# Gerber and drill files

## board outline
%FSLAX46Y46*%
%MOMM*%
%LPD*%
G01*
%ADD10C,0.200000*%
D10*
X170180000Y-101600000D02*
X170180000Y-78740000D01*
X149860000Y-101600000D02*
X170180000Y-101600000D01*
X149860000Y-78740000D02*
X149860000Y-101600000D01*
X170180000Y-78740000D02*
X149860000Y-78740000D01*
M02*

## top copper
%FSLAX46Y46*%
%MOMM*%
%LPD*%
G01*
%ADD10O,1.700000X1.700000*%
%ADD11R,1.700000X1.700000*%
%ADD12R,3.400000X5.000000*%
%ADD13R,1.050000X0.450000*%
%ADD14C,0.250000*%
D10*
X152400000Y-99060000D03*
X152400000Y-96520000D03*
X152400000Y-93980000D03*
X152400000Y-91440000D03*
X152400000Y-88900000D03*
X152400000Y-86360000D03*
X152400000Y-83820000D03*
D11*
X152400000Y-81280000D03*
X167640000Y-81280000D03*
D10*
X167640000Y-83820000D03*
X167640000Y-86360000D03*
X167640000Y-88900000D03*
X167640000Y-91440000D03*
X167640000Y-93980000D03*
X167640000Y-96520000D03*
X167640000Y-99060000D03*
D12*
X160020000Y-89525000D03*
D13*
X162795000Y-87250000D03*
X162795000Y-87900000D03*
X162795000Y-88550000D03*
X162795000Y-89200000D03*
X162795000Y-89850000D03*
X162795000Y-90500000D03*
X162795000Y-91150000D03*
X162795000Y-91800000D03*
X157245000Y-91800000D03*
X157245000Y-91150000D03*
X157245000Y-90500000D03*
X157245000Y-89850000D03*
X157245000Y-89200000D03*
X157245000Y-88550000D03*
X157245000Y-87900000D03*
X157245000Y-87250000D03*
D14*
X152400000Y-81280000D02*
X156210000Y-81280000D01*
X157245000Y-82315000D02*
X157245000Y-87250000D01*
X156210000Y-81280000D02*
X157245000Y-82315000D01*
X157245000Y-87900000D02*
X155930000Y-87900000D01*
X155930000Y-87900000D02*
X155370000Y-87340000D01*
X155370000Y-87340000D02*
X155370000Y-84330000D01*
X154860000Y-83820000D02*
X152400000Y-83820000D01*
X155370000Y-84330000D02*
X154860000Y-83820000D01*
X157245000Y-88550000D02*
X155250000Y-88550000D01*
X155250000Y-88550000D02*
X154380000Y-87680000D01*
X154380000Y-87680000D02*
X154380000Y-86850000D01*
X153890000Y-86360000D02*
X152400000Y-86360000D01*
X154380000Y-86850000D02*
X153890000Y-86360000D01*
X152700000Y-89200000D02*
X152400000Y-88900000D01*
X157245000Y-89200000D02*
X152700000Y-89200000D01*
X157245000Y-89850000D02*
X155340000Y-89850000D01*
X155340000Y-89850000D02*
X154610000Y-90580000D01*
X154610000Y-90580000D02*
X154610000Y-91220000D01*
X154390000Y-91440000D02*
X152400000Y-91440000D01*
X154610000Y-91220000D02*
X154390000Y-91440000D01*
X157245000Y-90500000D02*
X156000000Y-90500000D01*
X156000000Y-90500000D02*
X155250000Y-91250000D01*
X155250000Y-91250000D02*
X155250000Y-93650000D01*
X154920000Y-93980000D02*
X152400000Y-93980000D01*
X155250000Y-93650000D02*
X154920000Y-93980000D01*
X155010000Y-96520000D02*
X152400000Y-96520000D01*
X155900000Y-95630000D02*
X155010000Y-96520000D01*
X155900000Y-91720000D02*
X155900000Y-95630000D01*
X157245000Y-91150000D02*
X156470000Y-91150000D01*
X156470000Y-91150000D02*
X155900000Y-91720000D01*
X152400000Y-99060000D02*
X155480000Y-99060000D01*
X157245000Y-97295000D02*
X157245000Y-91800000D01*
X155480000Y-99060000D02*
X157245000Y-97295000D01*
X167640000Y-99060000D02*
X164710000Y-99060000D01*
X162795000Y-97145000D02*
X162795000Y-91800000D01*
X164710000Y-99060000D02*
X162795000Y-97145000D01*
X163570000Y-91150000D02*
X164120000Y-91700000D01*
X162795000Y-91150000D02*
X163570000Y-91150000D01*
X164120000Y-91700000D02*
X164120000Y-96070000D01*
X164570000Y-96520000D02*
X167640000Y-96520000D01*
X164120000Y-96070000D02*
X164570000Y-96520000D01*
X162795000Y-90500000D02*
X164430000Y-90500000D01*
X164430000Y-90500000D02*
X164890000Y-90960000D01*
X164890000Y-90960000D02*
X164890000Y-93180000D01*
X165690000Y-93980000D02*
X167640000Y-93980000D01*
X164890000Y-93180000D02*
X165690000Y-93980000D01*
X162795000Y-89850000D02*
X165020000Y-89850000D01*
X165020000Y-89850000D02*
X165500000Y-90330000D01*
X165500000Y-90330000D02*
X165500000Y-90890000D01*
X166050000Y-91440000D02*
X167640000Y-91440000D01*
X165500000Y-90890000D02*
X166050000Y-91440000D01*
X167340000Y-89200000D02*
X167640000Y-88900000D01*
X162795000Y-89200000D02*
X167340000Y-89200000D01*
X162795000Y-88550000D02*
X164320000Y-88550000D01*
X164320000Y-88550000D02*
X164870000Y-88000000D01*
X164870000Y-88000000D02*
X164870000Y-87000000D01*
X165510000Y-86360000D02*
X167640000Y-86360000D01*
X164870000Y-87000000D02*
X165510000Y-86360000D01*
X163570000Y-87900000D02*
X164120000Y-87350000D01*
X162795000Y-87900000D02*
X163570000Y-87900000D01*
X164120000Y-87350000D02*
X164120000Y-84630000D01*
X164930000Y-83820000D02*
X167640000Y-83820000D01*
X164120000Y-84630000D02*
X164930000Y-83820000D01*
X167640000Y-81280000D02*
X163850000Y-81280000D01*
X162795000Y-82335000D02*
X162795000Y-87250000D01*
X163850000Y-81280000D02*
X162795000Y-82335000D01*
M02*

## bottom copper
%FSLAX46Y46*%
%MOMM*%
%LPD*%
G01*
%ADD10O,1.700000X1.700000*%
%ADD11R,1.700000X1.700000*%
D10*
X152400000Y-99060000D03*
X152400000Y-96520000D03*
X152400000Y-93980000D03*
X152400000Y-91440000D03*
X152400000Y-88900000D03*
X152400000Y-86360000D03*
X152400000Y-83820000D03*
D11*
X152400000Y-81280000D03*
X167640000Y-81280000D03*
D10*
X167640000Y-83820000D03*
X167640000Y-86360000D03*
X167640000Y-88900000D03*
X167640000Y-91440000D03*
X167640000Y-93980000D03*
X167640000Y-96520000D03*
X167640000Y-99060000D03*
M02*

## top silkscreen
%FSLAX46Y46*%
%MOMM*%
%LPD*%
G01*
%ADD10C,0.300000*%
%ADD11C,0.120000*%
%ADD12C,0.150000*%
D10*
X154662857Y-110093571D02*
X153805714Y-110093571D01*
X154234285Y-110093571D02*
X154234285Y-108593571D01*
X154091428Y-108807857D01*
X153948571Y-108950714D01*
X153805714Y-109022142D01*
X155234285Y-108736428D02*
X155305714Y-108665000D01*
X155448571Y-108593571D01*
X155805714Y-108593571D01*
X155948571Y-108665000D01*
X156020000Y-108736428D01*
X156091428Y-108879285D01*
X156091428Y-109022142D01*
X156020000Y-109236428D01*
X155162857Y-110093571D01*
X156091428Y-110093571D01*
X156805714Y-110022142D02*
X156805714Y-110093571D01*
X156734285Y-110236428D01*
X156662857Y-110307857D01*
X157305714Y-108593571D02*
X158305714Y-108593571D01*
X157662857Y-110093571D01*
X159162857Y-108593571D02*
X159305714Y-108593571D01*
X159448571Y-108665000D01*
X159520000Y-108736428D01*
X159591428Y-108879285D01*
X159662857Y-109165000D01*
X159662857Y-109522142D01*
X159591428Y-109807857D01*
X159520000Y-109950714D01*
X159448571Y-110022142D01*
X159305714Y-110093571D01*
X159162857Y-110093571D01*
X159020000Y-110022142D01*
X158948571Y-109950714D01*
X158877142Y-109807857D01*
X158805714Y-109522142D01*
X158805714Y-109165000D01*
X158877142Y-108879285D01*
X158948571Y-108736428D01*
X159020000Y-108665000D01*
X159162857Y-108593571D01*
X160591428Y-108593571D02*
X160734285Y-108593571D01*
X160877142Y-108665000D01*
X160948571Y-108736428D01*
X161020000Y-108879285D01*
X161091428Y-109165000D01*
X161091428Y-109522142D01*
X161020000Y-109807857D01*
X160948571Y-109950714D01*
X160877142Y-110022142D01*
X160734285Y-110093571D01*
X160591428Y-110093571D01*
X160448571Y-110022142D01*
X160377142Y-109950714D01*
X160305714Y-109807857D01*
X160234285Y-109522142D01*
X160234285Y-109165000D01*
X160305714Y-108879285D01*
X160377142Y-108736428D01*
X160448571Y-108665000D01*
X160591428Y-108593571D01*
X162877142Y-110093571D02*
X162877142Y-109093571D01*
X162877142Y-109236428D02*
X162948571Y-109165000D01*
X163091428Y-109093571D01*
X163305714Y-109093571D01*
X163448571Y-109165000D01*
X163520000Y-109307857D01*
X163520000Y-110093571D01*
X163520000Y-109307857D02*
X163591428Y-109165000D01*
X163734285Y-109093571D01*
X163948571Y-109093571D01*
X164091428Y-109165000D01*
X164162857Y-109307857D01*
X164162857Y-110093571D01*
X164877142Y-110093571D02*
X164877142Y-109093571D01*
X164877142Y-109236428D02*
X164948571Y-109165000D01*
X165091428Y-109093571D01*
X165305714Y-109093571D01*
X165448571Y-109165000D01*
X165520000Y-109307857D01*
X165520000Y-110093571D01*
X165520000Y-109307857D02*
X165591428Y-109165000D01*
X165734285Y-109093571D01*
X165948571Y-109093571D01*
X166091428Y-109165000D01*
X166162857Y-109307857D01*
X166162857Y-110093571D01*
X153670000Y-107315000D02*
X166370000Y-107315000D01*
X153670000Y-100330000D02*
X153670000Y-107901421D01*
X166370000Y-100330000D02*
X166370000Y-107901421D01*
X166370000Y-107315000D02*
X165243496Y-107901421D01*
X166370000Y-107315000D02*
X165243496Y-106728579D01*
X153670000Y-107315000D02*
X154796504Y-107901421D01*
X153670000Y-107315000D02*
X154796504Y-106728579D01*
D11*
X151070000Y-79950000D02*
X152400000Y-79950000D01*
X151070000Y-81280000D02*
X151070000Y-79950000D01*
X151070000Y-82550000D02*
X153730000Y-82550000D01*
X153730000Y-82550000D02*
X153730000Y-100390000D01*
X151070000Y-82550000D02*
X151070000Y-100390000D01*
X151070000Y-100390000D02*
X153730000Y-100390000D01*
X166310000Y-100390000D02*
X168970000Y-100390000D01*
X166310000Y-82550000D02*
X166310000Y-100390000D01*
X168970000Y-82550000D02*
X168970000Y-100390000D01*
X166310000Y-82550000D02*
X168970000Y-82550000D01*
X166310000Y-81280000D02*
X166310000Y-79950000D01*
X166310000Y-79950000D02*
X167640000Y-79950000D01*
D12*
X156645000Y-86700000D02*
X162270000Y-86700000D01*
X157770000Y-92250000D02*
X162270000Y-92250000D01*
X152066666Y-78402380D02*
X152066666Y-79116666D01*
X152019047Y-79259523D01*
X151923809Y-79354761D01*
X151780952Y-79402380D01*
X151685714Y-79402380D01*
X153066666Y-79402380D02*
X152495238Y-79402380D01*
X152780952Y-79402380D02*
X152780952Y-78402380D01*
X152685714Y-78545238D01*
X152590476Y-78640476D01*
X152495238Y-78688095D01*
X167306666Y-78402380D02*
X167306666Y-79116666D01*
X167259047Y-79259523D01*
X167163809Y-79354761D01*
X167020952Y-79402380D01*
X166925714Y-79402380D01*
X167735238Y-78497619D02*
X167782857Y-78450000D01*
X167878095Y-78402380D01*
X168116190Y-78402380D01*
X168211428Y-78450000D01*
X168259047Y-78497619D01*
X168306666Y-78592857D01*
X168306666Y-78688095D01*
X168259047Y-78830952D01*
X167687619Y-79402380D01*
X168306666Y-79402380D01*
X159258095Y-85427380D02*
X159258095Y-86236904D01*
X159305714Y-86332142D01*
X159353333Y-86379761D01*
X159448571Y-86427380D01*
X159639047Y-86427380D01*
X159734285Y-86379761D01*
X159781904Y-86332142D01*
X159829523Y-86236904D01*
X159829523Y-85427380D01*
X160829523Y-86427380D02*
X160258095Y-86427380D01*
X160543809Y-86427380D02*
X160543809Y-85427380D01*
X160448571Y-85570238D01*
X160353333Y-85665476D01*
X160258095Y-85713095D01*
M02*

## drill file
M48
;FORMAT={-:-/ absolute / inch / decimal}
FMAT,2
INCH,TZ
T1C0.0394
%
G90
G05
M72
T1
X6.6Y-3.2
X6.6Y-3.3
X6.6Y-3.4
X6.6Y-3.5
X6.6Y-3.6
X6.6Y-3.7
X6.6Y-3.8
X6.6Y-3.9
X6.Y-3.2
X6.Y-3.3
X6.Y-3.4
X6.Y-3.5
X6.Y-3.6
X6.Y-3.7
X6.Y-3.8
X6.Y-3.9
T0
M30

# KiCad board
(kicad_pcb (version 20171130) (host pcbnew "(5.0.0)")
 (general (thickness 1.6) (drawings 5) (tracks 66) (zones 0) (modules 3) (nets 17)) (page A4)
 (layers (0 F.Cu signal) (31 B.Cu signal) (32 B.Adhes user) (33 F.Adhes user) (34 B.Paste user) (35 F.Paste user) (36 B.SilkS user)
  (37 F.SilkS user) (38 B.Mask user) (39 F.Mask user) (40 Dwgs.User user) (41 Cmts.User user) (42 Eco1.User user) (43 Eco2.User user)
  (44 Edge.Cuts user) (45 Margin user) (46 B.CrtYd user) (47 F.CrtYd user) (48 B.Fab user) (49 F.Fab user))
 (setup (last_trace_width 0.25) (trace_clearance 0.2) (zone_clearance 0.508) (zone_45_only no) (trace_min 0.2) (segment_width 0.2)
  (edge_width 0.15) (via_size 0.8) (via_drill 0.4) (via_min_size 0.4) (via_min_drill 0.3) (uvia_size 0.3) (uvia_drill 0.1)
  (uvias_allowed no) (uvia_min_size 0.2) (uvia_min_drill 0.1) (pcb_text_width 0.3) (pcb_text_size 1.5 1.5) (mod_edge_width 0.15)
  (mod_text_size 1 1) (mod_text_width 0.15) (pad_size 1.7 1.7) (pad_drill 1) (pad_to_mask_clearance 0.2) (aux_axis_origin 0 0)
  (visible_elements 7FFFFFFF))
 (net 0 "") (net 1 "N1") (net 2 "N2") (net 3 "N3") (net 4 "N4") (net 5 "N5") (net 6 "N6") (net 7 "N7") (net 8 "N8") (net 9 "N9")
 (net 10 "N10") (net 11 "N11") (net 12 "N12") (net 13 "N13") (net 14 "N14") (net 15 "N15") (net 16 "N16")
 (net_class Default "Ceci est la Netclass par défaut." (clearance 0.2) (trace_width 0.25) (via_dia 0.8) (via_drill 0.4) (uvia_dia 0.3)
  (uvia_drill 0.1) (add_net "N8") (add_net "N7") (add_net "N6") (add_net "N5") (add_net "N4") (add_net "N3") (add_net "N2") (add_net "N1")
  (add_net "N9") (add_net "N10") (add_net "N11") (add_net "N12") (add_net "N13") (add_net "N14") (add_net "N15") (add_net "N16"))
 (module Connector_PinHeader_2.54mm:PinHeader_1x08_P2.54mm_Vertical (layer F.Cu) (at 152.4 81.28)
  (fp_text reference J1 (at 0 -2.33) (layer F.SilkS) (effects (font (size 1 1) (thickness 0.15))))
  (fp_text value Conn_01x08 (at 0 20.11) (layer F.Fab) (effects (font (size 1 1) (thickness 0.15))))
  (fp_line (start -1.33 -1.33) (end 0 -1.33) (layer F.SilkS) (width 0.12))
  (fp_line (start -1.33 0) (end -1.33 -1.33) (layer F.SilkS) (width 0.12))
  (fp_line (start -1.33 1.27) (end 1.33 1.27) (layer F.SilkS) (width 0.12))
  (fp_line (start 1.33 1.27) (end 1.33 19.11) (layer F.SilkS) (width 0.12))
  (fp_line (start -1.33 1.27) (end -1.33 19.11) (layer F.SilkS) (width 0.12))
  (fp_line (start -1.33 19.11) (end 1.33 19.11) (layer F.SilkS) (width 0.12))
  (pad 8 thru_hole oval (at 0 17.78) (size 1.7 1.7) (drill 1) (layers *.Cu *.Mask) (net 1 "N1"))
  (pad 7 thru_hole oval (at 0 15.24) (size 1.7 1.7) (drill 1) (layers *.Cu *.Mask) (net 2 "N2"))
  (pad 6 thru_hole oval (at 0 12.7) (size 1.7 1.7) (drill 1) (layers *.Cu *.Mask) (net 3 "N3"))
  (pad 5 thru_hole oval (at 0 10.16) (size 1.7 1.7) (drill 1) (layers *.Cu *.Mask) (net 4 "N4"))
  (pad 4 thru_hole oval (at 0 7.62) (size 1.7 1.7) (drill 1) (layers *.Cu *.Mask) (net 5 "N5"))
  (pad 3 thru_hole oval (at 0 5.08) (size 1.7 1.7) (drill 1) (layers *.Cu *.Mask) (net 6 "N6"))
  (pad 2 thru_hole oval (at 0 2.54) (size 1.7 1.7) (drill 1) (layers *.Cu *.Mask) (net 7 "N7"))
  (pad 1 thru_hole rect (at 0 0) (size 1.7 1.7) (drill 1) (layers *.Cu *.Mask) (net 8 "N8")))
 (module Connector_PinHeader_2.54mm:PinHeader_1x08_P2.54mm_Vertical (layer F.Cu) (at 167.64 81.28)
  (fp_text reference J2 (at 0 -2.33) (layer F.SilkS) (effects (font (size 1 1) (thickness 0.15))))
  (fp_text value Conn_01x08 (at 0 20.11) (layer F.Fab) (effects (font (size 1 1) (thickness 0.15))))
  (fp_line (start -1.33 19.11) (end 1.33 19.11) (layer F.SilkS) (width 0.12))
  (fp_line (start -1.33 1.27) (end -1.33 19.11) (layer F.SilkS) (width 0.12))
  (fp_line (start 1.33 1.27) (end 1.33 19.11) (layer F.SilkS) (width 0.12))
  (fp_line (start -1.33 1.27) (end 1.33 1.27) (layer F.SilkS) (width 0.12))
  (fp_line (start -1.33 0) (end -1.33 -1.33) (layer F.SilkS) (width 0.12))
  (fp_line (start -1.33 -1.33) (end 0 -1.33) (layer F.SilkS) (width 0.12))
  (pad 1 thru_hole rect (at 0 0) (size 1.7 1.7) (drill 1) (layers *.Cu *.Mask) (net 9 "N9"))
  (pad 2 thru_hole oval (at 0 2.54) (size 1.7 1.7) (drill 1) (layers *.Cu *.Mask) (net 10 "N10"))
  (pad 3 thru_hole oval (at 0 5.08) (size 1.7 1.7) (drill 1) (layers *.Cu *.Mask) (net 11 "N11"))
  (pad 4 thru_hole oval (at 0 7.62) (size 1.7 1.7) (drill 1) (layers *.Cu *.Mask) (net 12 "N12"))
  (pad 5 thru_hole oval (at 0 10.16) (size 1.7 1.7) (drill 1) (layers *.Cu *.Mask) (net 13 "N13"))
  (pad 6 thru_hole oval (at 0 12.7) (size 1.7 1.7) (drill 1) (layers *.Cu *.Mask) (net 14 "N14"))
  (pad 7 thru_hole oval (at 0 15.24) (size 1.7 1.7) (drill 1) (layers *.Cu *.Mask) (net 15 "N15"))
  (pad 8 thru_hole oval (at 0 17.78) (size 1.7 1.7) (drill 1) (layers *.Cu *.Mask) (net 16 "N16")))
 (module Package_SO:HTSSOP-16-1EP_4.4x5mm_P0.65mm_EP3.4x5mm (layer F.Cu) (at 160.02 89.525)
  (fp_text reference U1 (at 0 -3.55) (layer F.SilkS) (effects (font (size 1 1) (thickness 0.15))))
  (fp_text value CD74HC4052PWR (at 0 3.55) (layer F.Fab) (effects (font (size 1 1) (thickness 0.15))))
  (fp_line (start -3.375 -2.825) (end 2.25 -2.825) (layer F.SilkS) (width 0.15))
  (fp_line (start -2.25 2.725) (end 2.25 2.725) (layer F.SilkS) (width 0.15))
  (pad "" smd rect (at -1.1334 1.875) (size 0.88 1.05) (layers F.Paste))
  (pad "" smd rect (at 0 1.875) (size 0.88 1.05) (layers F.Paste))
  (pad "" smd rect (at 1.1334 1.875) (size 0.88 1.05) (layers F.Paste))
  (pad "" smd rect (at -1.1334 0.625) (size 0.88 1.05) (layers F.Paste))
  (pad "" smd rect (at 0 0.625) (size 0.88 1.05) (layers F.Paste))
  (pad "" smd rect (at 1.1334 0.625) (size 0.88 1.05) (layers F.Paste))
  (pad "" smd rect (at -1.1334 -0.625) (size 0.88 1.05) (layers F.Paste))
  (pad "" smd rect (at 0 -0.625) (size 0.88 1.05) (layers F.Paste))
  (pad "" smd rect (at 1.1334 -0.625) (size 0.88 1.05) (layers F.Paste))
  (pad "" smd rect (at 1.1334 -1.875) (size 0.88 1.05) (layers F.Paste))
  (pad "" smd rect (at 0 -1.875) (size 0.88 1.05) (layers F.Paste))
  (pad "" smd rect (at -1.1334 -1.875) (size 0.88 1.05) (layers F.Paste)) (pad 17 smd rect (at 0 0) (size 3.4 5) (layers F.Cu F.Mask))
  (pad 16 smd rect (at 2.775 -2.275) (size 1.05 0.45) (layers F.Cu F.Paste F.Mask) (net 9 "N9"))
  (pad 15 smd rect (at 2.775 -1.625) (size 1.05 0.45) (layers F.Cu F.Paste F.Mask) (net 10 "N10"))
  (pad 14 smd rect (at 2.775 -0.975) (size 1.05 0.45) (layers F.Cu F.Paste F.Mask) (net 11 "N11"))
  (pad 13 smd rect (at 2.775 -0.325) (size 1.05 0.45) (layers F.Cu F.Paste F.Mask) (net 12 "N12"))
  (pad 12 smd rect (at 2.775 0.325) (size 1.05 0.45) (layers F.Cu F.Paste F.Mask) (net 13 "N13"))
  (pad 11 smd rect (at 2.775 0.975) (size 1.05 0.45) (layers F.Cu F.Paste F.Mask) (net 14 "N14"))
  (pad 10 smd rect (at 2.775 1.625) (size 1.05 0.45) (layers F.Cu F.Paste F.Mask) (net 15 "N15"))
  (pad 9 smd rect (at 2.775 2.275) (size 1.05 0.45) (layers F.Cu F.Paste F.Mask) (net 16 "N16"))
  (pad 8 smd rect (at -2.775 2.275) (size 1.05 0.45) (layers F.Cu F.Paste F.Mask) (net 1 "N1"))
  (pad 7 smd rect (at -2.775 1.625) (size 1.05 0.45) (layers F.Cu F.Paste F.Mask) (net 2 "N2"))
  (pad 6 smd rect (at -2.775 0.975) (size 1.05 0.45) (layers F.Cu F.Paste F.Mask) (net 3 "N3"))
  (pad 5 smd rect (at -2.775 0.325) (size 1.05 0.45) (layers F.Cu F.Paste F.Mask) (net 4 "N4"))
  (pad 4 smd rect (at -2.775 -0.325) (size 1.05 0.45) (layers F.Cu F.Paste F.Mask) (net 5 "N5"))
  (pad 3 smd rect (at -2.775 -0.975) (size 1.05 0.45) (layers F.Cu F.Paste F.Mask) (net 6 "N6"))
  (pad 2 smd rect (at -2.775 -1.625) (size 1.05 0.45) (layers F.Cu F.Paste F.Mask) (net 7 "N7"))
  (pad 1 smd rect (at -2.775 -2.275) (size 1.05 0.45) (layers F.Cu F.Paste F.Mask) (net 8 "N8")))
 (gr_line (start 170.18 101.6) (end 170.18 78.74) (layer Edge.Cuts) (width 0.2))
 (gr_line (start 149.86 101.6) (end 170.18 101.6) (layer Edge.Cuts) (width 0.2))
 (gr_line (start 149.86 78.74) (end 149.86 101.6) (layer Edge.Cuts) (width 0.2))
 (gr_line (start 170.18 78.74) (end 149.86 78.74) (layer Edge.Cuts) (width 0.2))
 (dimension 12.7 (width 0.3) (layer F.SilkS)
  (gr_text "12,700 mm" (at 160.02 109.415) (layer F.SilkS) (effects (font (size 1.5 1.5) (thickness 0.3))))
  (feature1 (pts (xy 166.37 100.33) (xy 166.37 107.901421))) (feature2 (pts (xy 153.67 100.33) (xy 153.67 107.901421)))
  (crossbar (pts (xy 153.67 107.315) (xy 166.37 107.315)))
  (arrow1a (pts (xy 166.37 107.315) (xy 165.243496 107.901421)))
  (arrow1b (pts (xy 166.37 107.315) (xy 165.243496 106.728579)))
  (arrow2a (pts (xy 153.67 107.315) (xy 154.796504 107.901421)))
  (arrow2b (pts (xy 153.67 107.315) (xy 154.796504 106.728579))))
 (segment (start 152.4 81.28) (end 156.21 81.28) (width 0.25) (layer F.Cu) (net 8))
 (segment (start 157.245 82.315) (end 157.245 87.25) (width 0.25) (layer F.Cu) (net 8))
 (segment (start 156.21 81.28) (end 157.245 82.315) (width 0.25) (layer F.Cu) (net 8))
 (segment (start 157.245 87.9) (end 155.93 87.9) (width 0.25) (layer F.Cu) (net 7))
 (segment (start 155.93 87.9) (end 155.37 87.34) (width 0.25) (layer F.Cu) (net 7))
 (segment (start 155.37 87.34) (end 155.37 84.33) (width 0.25) (layer F.Cu) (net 7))
 (segment (start 154.86 83.82) (end 152.4 83.82) (width 0.25) (layer F.Cu) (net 7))
 (segment (start 155.37 84.33) (end 154.86 83.82) (width 0.25) (layer F.Cu) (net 7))
 (segment (start 157.245 88.55) (end 155.25 88.55) (width 0.25) (layer F.Cu) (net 6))
 (segment (start 155.25 88.55) (end 154.38 87.68) (width 0.25) (layer F.Cu) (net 6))
 (segment (start 154.38 87.68) (end 154.38 86.85) (width 0.25) (layer F.Cu) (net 6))
 (segment (start 153.89 86.36) (end 152.4 86.36) (width 0.25) (layer F.Cu) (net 6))
 (segment (start 154.38 86.85) (end 153.89 86.36) (width 0.25) (layer F.Cu) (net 6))
 (segment (start 152.7 89.2) (end 152.4 88.9) (width 0.25) (layer F.Cu) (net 5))
 (segment (start 157.245 89.2) (end 152.7 89.2) (width 0.25) (layer F.Cu) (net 5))
 (segment (start 157.245 89.85) (end 155.34 89.85) (width 0.25) (layer F.Cu) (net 4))
 (segment (start 155.34 89.85) (end 154.61 90.58) (width 0.25) (layer F.Cu) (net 4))
 (segment (start 154.61 90.58) (end 154.61 91.22) (width 0.25) (layer F.Cu) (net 4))
 (segment (start 154.39 91.44) (end 152.4 91.44) (width 0.25) (layer F.Cu) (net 4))
 (segment (start 154.61 91.22) (end 154.39 91.44) (width 0.25) (layer F.Cu) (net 4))
 (segment (start 157.245 90.5) (end 156 90.5) (width 0.25) (layer F.Cu) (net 3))
 (segment (start 156 90.5) (end 155.25 91.25) (width 0.25) (layer F.Cu) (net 3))
 (segment (start 155.25 91.25) (end 155.25 93.65) (width 0.25) (layer F.Cu) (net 3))
 (segment (start 154.92 93.98) (end 152.4 93.98) (width 0.25) (layer F.Cu) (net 3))
 (segment (start 155.25 93.65) (end 154.92 93.98) (width 0.25) (layer F.Cu) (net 3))
 (segment (start 155.01 96.52) (end 152.4 96.52) (width 0.25) (layer F.Cu) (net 2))
 (segment (start 155.9 95.63) (end 155.01 96.52) (width 0.25) (layer F.Cu) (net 2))
 (segment (start 155.9 91.72) (end 155.9 95.63) (width 0.25) (layer F.Cu) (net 2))
 (segment (start 157.245 91.15) (end 156.47 91.15) (width 0.25) (layer F.Cu) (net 2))
 (segment (start 156.47 91.15) (end 155.9 91.72) (width 0.25) (layer F.Cu) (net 2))
 (segment (start 152.4 99.06) (end 155.48 99.06) (width 0.25) (layer F.Cu) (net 1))
 (segment (start 157.245 97.295) (end 157.245 91.8) (width 0.25) (layer F.Cu) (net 1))
 (segment (start 155.48 99.06) (end 157.245 97.295) (width 0.25) (layer F.Cu) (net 1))
 (segment (start 167.64 99.06) (end 164.71 99.06) (width 0.25) (layer F.Cu) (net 16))
 (segment (start 162.795 97.145) (end 162.795 91.8) (width 0.25) (layer F.Cu) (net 16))
 (segment (start 164.71 99.06) (end 162.795 97.145) (width 0.25) (layer F.Cu) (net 16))
 (segment (start 163.57 91.15) (end 164.12 91.7) (width 0.25) (layer F.Cu) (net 15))
 (segment (start 162.795 91.15) (end 163.57 91.15) (width 0.25) (layer F.Cu) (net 15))
 (segment (start 164.12 91.7) (end 164.12 96.07) (width 0.25) (layer F.Cu) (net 15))
 (segment (start 164.57 96.52) (end 167.64 96.52) (width 0.25) (layer F.Cu) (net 15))
 (segment (start 164.12 96.07) (end 164.57 96.52) (width 0.25) (layer F.Cu) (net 15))
 (segment (start 162.795 90.5) (end 164.43 90.5) (width 0.25) (layer F.Cu) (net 14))
 (segment (start 164.43 90.5) (end 164.89 90.96) (width 0.25) (layer F.Cu) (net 14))
 (segment (start 164.89 90.96) (end 164.89 93.18) (width 0.25) (layer F.Cu) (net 14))
 (segment (start 165.69 93.98) (end 167.64 93.98) (width 0.25) (layer F.Cu) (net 14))
 (segment (start 164.89 93.18) (end 165.69 93.98) (width 0.25) (layer F.Cu) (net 14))
 (segment (start 162.795 89.85) (end 165.02 89.85) (width 0.25) (layer F.Cu) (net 13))
 (segment (start 165.02 89.85) (end 165.5 90.33) (width 0.25) (layer F.Cu) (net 13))
 (segment (start 165.5 90.33) (end 165.5 90.89) (width 0.25) (layer F.Cu) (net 13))
 (segment (start 166.05 91.44) (end 167.64 91.44) (width 0.25) (layer F.Cu) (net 13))
 (segment (start 165.5 90.89) (end 166.05 91.44) (width 0.25) (layer F.Cu) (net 13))
 (segment (start 167.34 89.2) (end 167.64 88.9) (width 0.25) (layer F.Cu) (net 12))
 (segment (start 162.795 89.2) (end 167.34 89.2) (width 0.25) (layer F.Cu) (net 12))
 (segment (start 162.795 88.55) (end 164.32 88.55) (width 0.25) (layer F.Cu) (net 11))
 (segment (start 164.32 88.55) (end 164.87 88) (width 0.25) (layer F.Cu) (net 11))
 (segment (start 164.87 88) (end 164.87 87) (width 0.25) (layer F.Cu) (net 11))
 (segment (start 165.51 86.36) (end 167.64 86.36) (width 0.25) (layer F.Cu) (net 11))
 (segment (start 164.87 87) (end 165.51 86.36) (width 0.25) (layer F.Cu) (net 11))
 (segment (start 163.57 87.9) (end 164.12 87.35) (width 0.25) (layer F.Cu) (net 10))
 (segment (start 162.795 87.9) (end 163.57 87.9) (width 0.25) (layer F.Cu) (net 10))
 (segment (start 164.12 87.35) (end 164.12 84.63) (width 0.25) (layer F.Cu) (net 10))
 (segment (start 164.93 83.82) (end 167.64 83.82) (width 0.25) (layer F.Cu) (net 10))
 (segment (start 164.12 84.63) (end 164.93 83.82) (width 0.25) (layer F.Cu) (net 10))
 (segment (start 167.64 81.28) (end 163.85 81.28) (width 0.25) (layer F.Cu) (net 9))
 (segment (start 162.795 82.335) (end 162.795 87.25) (width 0.25) (layer F.Cu) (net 9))
 (segment (start 163.85 81.28) (end 162.795 82.335) (width 0.25) (layer F.Cu) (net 9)))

